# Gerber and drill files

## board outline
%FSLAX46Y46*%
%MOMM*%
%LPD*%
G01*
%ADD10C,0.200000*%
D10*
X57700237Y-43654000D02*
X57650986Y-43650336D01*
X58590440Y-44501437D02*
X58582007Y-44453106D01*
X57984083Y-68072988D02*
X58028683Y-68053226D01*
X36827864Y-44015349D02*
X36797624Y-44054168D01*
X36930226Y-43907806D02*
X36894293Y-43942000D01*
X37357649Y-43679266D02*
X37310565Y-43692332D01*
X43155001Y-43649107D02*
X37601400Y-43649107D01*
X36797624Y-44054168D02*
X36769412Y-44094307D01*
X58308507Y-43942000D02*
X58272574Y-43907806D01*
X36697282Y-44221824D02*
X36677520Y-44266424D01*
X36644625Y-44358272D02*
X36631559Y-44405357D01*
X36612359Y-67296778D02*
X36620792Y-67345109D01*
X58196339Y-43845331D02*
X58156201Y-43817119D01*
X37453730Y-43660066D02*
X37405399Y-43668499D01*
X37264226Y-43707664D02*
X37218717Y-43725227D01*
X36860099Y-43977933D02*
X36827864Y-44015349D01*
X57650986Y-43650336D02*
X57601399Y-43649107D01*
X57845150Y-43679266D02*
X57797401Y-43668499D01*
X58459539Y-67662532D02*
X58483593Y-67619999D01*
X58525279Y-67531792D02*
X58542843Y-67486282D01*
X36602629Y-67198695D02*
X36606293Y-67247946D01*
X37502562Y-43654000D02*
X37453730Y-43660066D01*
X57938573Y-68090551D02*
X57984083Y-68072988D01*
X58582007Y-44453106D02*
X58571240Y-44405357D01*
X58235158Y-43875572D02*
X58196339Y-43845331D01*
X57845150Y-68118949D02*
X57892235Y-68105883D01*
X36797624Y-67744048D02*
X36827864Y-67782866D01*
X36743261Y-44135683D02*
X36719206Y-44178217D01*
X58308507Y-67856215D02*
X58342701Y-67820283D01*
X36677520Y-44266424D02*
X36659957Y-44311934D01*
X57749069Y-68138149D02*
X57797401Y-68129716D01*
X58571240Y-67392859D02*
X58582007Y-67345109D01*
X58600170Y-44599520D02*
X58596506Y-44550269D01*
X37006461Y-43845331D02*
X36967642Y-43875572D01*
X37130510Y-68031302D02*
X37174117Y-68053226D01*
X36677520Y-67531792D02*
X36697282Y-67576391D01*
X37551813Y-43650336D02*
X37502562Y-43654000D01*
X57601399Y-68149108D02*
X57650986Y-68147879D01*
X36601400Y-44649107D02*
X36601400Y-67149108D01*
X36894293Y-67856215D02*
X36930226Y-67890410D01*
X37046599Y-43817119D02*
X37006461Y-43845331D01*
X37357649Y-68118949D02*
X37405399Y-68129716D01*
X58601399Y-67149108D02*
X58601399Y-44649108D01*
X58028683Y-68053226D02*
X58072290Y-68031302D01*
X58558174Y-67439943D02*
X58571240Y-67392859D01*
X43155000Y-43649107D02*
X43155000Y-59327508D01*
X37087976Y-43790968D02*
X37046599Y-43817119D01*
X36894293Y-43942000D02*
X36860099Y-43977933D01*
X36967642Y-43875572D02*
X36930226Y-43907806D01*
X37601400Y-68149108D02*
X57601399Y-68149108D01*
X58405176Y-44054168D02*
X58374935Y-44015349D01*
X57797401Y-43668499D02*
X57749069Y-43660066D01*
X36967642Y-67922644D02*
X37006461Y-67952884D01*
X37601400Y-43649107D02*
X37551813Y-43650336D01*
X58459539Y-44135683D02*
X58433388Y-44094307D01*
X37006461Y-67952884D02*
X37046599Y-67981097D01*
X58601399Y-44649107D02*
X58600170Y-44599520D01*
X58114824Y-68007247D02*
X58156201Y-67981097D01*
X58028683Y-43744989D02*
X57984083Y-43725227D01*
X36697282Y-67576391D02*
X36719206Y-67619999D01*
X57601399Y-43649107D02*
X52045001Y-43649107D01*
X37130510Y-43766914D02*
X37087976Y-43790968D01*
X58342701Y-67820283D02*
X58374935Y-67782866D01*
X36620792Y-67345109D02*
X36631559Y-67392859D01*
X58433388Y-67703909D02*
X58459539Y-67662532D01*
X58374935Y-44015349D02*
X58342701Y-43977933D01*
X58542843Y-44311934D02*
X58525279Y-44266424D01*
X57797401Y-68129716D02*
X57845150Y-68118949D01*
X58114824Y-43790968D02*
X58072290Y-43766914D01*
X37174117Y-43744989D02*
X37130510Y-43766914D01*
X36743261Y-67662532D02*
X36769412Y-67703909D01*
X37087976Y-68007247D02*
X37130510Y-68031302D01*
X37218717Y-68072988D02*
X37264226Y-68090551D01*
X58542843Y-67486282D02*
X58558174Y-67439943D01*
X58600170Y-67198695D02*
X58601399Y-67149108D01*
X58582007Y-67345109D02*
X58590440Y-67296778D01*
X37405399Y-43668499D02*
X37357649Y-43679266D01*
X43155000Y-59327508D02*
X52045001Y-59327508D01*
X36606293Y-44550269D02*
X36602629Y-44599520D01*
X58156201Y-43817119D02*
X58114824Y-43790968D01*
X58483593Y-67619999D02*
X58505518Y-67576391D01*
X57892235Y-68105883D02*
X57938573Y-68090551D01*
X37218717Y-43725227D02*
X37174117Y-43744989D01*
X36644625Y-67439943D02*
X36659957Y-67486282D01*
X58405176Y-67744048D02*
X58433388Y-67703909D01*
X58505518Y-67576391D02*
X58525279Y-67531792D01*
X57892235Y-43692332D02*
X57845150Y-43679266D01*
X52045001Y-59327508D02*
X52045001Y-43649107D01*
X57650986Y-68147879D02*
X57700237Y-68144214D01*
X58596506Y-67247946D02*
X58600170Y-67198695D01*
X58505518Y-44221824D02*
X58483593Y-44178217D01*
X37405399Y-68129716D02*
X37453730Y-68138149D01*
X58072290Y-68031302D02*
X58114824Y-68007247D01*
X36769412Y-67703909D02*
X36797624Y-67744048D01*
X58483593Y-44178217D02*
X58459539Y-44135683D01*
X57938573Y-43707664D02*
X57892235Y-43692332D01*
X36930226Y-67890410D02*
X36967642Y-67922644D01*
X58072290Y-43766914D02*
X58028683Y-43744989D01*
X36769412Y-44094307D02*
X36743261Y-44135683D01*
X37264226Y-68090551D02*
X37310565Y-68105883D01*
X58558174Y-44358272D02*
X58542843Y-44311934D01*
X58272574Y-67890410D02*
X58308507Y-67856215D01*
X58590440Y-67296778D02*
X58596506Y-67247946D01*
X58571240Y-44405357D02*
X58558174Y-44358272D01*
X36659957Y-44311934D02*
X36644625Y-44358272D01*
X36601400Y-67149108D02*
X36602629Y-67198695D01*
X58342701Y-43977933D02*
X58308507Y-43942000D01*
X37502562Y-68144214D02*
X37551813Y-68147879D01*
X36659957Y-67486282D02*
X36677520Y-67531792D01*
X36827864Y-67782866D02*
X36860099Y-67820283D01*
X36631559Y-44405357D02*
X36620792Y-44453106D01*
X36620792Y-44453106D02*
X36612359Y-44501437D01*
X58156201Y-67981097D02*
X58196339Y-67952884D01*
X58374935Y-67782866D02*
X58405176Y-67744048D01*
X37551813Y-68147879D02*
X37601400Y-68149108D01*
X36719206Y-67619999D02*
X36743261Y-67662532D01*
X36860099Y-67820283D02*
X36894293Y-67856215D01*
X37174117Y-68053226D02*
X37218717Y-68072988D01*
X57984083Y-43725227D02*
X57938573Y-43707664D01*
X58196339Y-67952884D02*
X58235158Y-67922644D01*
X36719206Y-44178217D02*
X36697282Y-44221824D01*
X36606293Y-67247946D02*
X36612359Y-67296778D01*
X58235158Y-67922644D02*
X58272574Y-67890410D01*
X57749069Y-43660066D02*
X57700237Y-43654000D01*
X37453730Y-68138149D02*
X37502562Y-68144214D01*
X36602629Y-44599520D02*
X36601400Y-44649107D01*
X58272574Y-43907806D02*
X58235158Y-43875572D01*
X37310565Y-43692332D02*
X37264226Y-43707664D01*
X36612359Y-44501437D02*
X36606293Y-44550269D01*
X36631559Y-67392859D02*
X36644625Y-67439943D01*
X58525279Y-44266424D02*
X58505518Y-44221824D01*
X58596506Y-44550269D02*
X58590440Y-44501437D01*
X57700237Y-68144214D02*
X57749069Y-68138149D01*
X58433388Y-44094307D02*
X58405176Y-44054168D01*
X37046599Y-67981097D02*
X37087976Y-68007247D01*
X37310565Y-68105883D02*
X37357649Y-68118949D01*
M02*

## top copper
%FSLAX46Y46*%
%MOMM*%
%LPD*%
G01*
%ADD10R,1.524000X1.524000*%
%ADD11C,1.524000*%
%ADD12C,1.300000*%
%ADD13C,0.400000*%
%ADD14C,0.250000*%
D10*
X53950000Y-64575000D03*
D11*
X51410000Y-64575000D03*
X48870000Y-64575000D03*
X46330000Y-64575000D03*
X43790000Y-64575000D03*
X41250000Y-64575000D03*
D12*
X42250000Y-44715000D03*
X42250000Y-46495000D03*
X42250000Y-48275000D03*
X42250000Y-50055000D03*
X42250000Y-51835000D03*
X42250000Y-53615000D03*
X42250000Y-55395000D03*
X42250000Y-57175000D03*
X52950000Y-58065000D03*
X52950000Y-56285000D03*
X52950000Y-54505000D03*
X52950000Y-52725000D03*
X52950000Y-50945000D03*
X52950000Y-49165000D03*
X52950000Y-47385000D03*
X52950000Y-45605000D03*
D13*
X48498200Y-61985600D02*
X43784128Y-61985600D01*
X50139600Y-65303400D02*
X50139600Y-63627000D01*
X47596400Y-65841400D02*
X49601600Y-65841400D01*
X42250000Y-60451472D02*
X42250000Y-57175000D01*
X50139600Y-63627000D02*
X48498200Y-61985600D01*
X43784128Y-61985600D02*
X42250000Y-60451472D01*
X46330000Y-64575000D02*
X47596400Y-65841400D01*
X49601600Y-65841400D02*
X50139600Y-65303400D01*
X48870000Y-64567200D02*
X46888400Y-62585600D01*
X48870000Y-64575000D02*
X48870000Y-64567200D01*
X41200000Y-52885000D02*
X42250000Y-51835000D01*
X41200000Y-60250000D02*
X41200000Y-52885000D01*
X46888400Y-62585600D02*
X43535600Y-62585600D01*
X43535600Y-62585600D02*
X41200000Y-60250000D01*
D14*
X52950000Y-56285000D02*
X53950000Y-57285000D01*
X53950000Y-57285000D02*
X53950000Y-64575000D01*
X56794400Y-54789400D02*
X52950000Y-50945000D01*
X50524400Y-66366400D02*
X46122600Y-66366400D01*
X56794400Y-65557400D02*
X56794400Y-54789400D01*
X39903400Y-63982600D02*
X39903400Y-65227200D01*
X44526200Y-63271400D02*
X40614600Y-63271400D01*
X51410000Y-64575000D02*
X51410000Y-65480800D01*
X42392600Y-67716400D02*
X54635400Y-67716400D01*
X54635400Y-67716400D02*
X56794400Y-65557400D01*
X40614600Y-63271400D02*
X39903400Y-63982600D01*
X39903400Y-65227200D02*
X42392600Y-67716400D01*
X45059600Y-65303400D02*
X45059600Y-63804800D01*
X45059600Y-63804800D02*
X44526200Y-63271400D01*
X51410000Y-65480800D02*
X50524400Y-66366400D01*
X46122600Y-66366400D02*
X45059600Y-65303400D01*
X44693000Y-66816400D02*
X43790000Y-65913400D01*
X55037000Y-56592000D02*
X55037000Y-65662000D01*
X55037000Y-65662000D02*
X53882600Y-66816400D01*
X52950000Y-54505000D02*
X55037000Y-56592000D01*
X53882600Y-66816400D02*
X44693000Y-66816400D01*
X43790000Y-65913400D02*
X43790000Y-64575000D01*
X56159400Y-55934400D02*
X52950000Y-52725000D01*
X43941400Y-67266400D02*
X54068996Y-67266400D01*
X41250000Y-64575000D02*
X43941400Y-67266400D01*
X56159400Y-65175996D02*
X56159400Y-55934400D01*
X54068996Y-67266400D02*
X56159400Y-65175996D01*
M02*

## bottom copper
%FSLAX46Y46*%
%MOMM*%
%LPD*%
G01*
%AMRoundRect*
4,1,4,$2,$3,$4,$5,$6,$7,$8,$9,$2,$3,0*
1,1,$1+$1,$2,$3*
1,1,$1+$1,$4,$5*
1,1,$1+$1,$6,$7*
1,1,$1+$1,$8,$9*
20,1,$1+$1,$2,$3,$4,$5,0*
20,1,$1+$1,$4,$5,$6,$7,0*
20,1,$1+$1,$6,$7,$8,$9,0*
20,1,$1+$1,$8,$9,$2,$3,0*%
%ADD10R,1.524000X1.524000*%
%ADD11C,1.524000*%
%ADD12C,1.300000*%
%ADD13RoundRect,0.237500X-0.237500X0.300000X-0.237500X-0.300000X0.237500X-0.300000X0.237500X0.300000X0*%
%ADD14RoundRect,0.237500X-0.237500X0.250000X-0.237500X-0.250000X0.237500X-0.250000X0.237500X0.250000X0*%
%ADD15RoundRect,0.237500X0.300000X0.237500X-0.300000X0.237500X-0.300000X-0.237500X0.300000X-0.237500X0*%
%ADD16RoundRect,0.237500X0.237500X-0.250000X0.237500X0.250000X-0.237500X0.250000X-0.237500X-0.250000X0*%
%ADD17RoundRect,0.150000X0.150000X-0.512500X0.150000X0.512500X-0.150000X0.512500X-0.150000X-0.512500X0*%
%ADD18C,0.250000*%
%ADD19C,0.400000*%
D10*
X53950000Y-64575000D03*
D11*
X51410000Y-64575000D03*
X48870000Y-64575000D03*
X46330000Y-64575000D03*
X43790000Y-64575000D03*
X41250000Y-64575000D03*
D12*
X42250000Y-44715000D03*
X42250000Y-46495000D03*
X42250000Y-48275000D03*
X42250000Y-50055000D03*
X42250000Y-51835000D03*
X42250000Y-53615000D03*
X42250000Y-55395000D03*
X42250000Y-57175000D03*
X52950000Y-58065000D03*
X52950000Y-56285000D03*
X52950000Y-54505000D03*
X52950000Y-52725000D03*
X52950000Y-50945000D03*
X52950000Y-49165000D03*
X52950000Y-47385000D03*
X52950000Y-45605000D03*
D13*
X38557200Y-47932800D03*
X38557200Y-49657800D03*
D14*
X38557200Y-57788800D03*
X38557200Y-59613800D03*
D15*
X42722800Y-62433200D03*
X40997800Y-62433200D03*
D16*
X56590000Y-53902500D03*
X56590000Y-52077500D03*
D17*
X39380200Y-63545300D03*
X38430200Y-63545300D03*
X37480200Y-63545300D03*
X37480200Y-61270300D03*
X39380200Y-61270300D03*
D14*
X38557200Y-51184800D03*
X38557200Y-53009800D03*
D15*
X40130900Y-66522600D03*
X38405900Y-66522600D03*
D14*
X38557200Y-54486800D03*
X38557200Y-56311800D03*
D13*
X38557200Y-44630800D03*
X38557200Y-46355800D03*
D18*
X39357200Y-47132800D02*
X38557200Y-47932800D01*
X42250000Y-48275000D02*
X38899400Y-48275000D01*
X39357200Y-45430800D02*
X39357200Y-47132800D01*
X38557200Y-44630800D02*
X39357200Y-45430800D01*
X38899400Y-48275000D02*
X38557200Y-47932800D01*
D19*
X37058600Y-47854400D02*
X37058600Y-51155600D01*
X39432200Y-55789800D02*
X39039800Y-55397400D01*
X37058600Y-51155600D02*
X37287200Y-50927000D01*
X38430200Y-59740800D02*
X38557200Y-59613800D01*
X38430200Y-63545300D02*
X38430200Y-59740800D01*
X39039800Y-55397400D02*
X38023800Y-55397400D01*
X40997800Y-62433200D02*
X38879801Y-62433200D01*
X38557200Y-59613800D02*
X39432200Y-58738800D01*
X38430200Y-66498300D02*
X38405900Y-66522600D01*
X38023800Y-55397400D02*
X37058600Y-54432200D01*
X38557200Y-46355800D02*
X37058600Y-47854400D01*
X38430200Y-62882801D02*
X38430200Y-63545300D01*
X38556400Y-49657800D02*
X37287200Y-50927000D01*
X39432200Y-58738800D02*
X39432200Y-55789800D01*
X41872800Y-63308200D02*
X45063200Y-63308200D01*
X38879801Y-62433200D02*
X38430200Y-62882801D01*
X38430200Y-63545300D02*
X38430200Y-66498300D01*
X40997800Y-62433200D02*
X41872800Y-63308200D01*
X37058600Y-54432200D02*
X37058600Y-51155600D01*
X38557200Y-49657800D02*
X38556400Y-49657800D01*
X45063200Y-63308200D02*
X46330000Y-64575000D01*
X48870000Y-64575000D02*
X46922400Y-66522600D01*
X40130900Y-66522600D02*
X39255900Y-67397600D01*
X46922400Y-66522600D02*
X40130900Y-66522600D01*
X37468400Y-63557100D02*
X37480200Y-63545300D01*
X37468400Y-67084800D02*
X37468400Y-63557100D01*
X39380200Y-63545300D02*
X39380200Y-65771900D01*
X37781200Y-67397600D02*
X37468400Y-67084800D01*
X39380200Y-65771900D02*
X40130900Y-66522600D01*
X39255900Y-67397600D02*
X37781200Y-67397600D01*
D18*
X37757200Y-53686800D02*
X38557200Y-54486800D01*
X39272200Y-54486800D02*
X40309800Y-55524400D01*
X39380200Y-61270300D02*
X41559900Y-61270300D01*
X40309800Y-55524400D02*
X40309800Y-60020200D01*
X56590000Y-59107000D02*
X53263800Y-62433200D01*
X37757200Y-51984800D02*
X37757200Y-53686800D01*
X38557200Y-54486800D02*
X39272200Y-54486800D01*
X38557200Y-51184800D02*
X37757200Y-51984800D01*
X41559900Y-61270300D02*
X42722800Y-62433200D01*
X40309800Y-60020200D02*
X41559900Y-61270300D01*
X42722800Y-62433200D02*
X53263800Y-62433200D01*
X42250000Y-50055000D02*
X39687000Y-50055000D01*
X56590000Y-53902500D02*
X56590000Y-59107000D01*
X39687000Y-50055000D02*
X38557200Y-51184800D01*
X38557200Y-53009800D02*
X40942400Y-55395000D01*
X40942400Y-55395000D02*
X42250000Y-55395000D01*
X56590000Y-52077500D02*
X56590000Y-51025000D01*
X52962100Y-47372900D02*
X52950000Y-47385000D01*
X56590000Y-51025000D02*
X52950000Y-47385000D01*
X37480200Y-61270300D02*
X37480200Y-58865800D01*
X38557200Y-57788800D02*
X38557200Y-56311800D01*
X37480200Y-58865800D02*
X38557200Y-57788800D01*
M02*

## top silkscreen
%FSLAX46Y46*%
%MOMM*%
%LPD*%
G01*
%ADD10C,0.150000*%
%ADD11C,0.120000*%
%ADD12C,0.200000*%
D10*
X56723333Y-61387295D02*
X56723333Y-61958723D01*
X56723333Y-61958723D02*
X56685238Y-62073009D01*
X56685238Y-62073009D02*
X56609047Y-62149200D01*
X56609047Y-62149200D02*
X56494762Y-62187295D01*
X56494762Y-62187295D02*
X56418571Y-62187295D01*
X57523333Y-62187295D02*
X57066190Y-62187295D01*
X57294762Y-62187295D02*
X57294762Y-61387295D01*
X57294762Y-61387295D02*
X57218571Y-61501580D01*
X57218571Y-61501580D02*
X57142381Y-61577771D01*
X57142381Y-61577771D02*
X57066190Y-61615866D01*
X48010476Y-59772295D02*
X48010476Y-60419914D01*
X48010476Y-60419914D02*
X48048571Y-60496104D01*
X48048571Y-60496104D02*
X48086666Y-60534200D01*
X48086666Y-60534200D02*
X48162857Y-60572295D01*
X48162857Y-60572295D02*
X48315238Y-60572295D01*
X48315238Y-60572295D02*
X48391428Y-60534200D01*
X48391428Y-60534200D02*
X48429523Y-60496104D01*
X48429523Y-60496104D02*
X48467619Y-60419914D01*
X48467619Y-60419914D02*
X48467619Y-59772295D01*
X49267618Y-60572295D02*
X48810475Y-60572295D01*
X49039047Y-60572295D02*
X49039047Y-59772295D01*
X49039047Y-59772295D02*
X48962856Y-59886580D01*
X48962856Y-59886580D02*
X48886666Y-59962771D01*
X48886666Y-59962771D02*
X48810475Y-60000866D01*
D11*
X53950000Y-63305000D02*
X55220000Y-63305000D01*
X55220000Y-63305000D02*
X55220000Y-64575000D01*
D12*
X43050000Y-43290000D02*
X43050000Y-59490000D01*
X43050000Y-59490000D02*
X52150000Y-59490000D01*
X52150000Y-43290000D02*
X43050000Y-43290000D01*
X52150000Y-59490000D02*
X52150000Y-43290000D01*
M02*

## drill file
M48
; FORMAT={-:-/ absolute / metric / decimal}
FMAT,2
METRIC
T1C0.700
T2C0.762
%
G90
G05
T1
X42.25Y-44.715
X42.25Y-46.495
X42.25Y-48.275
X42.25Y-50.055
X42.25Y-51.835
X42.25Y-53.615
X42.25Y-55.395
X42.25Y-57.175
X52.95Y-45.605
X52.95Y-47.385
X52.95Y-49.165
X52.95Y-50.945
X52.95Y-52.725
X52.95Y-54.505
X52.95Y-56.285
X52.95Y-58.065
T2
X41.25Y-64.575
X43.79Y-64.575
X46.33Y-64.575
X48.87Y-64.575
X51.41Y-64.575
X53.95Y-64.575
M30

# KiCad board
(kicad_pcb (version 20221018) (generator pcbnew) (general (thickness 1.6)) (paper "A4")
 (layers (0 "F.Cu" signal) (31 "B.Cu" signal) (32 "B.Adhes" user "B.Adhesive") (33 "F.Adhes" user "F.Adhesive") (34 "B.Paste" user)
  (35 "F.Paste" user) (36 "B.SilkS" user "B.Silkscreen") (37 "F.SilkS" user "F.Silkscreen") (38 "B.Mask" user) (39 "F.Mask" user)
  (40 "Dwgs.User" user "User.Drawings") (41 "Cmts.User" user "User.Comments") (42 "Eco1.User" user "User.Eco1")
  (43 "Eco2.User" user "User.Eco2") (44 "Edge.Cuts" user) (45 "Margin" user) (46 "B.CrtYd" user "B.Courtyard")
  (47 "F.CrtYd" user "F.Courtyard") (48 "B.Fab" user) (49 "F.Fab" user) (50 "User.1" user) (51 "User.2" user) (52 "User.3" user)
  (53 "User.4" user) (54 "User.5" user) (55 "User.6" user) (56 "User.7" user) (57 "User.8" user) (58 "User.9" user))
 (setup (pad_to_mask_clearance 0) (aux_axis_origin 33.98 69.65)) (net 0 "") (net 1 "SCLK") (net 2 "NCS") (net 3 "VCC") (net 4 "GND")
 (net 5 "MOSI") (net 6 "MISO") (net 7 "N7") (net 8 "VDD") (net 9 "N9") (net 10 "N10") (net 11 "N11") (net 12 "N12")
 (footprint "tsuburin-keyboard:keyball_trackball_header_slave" (layer "F.Cu") (at 43.59 62.995)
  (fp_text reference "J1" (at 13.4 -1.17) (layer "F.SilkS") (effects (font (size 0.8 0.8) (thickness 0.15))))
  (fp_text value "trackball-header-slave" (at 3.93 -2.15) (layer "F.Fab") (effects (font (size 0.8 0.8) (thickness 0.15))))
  (fp_line (start 10.36 0.31) (end 11.63 0.31) (stroke (width 0.12) (type solid)) (layer "F.SilkS"))
  (fp_line (start 11.63 0.31) (end 11.63 1.58) (stroke (width 0.12) (type solid)) (layer "F.SilkS"))
  (pad "1" thru_hole rect (at 10.36 1.58 270) (size 1.524 1.524) (drill 0.762) (layers "*.Cu" "*.Mask") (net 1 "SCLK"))
  (pad "2" thru_hole circle (at 7.82 1.58 270) (size 1.524 1.524) (drill 0.762) (layers "*.Cu" "*.Mask") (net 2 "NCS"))
  (pad "3" thru_hole circle (at 5.28 1.58 270) (size 1.524 1.524) (drill 0.762) (layers "*.Cu" "*.Mask") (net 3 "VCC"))
  (pad "4" thru_hole circle (at 2.74 1.58 270) (size 1.524 1.524) (drill 0.762) (layers "*.Cu" "*.Mask") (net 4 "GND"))
  (pad "5" thru_hole circle (at 0.2 1.58 270) (size 1.524 1.524) (drill 0.762) (layers "*.Cu" "*.Mask") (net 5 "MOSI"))
  (pad "6" thru_hole circle (at -2.34 1.58 270) (size 1.524 1.524) (drill 0.762) (layers "*.Cu" "*.Mask") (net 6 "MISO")))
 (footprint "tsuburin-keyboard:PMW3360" (layer "F.Cu") (at 47.6 51.39)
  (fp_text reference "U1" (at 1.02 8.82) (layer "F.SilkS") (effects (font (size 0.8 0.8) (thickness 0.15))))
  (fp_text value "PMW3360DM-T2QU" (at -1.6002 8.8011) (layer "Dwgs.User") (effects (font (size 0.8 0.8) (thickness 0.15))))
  (fp_line (start -4.55 -8.1) (end -4.55 8.1) (stroke (width 0.2) (type solid)) (layer "F.SilkS"))
  (fp_line (start -4.55 8.1) (end 4.55 8.1) (stroke (width 0.2) (type solid)) (layer "F.SilkS"))
  (fp_line (start 4.55 -8.1) (end -4.55 -8.1) (stroke (width 0.2) (type solid)) (layer "F.SilkS"))
  (fp_line (start 4.55 8.1) (end 4.55 -8.1) (stroke (width 0.2) (type solid)) (layer "F.SilkS"))
  (pad "1" thru_hole circle (at -5.35 -6.675) (size 1.3 1.3) (drill 0.7) (layers "*.Cu" "*.Mask") (solder_mask_margin 0.102))
  (pad "2" thru_hole circle (at -5.35 -4.895) (size 1.3 1.3) (drill 0.7) (layers "*.Cu" "*.Mask") (solder_mask_margin 0.102))
  (pad "3" thru_hole circle (at -5.35 -3.115) (size 1.3 1.3) (drill 0.7) (layers "*.Cu" "*.Mask") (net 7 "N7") (solder_mask_margin 0.102))
  (pad "4" thru_hole circle (at -5.35 -1.335) (size 1.3 1.3) (drill 0.7) (layers "*.Cu" "*.Mask") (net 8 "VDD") (solder_mask_margin 0.102))
  (pad "5" thru_hole circle (at -5.35 0.445) (size 1.3 1.3) (drill 0.7) (layers "*.Cu" "*.Mask") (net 3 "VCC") (solder_mask_margin 0.102))
  (pad "6" thru_hole circle (at -5.35 2.225) (size 1.3 1.3) (drill 0.7) (layers "*.Cu" "*.Mask") (solder_mask_margin 0.102))
  (pad "7" thru_hole circle (at -5.35 4.005) (size 1.3 1.3) (drill 0.7) (layers "*.Cu" "*.Mask") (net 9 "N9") (solder_mask_margin 0.102))
  (pad "8" thru_hole circle (at -5.35 5.785) (size 1.3 1.3) (drill 0.7) (layers "*.Cu" "*.Mask") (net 4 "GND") (solder_mask_margin 0.102))
  (pad "9" thru_hole circle (at 5.35 6.675) (size 1.3 1.3) (drill 0.7) (layers "*.Cu" "*.Mask") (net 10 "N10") (solder_mask_margin 0.102))
  (pad "10" thru_hole circle (at 5.35 4.895) (size 1.3 1.3) (drill 0.7) (layers "*.Cu" "*.Mask") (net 1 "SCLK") (solder_mask_margin 0.102))
  (pad "11" thru_hole circle (at 5.35 3.115) (size 1.3 1.3) (drill 0.7) (layers "*.Cu" "*.Mask") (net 5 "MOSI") (solder_mask_margin 0.102))
  (pad "12" thru_hole circle (at 5.35 1.335) (size 1.3 1.3) (drill 0.7) (layers "*.Cu" "*.Mask") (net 6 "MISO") (solder_mask_margin 0.102))
  (pad "13" thru_hole circle (at 5.35 -0.445) (size 1.3 1.3) (drill 0.7) (layers "*.Cu" "*.Mask") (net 2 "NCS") (solder_mask_margin 0.102))
  (pad "14" thru_hole circle (at 5.35 -2.225) (size 1.3 1.3) (drill 0.7) (layers "*.Cu" "*.Mask") (solder_mask_margin 0.102))
  (pad "15" thru_hole circle (at 5.35 -4.005) (size 1.3 1.3) (drill 0.7) (layers "*.Cu" "*.Mask") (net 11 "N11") (solder_mask_margin 0.102))
  (pad "16" thru_hole circle (at 5.35 -5.785) (size 1.3 1.3) (drill 0.7) (layers "*.Cu" "*.Mask") (solder_mask_margin 0.102))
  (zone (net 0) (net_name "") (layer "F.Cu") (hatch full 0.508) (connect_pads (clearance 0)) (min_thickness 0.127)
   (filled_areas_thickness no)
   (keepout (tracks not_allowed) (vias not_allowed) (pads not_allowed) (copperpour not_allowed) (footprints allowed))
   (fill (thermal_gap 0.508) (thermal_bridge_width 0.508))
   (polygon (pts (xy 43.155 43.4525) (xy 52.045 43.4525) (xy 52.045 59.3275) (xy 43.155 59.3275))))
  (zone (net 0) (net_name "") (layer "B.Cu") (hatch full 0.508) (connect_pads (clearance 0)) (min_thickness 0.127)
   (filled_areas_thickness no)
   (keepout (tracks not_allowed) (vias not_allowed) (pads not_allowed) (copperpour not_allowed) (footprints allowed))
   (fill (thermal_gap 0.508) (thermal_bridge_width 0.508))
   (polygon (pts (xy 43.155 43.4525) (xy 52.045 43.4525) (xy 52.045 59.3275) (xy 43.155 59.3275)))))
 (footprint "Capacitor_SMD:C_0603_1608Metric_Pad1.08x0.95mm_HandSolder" (layer "B.Cu") (at 38.5572 48.7953 -90)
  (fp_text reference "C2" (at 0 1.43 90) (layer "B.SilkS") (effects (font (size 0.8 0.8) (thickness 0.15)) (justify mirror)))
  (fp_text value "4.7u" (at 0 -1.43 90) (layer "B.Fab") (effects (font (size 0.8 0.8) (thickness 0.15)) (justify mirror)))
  (pad "1" smd roundrect (at -0.8625 0 270) (size 1.075 0.95) (layers "B.Cu" "B.Paste" "B.Mask") (roundrect_rratio 0.25) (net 7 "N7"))
  (pad "2" smd roundrect (at 0.8625 0 270) (size 1.075 0.95) (layers "B.Cu" "B.Paste" "B.Mask") (roundrect_rratio 0.25) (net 4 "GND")))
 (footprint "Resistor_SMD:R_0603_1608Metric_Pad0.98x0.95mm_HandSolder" (layer "B.Cu") (at 38.5572 58.7013 -90)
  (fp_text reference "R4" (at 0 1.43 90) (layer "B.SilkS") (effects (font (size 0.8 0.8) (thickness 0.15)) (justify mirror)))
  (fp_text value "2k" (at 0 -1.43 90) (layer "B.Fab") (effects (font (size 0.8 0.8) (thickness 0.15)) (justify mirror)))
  (pad "1" smd roundrect (at -0.9125 0 270) (size 0.975 0.95) (layers "B.Cu" "B.Paste" "B.Mask") (roundrect_rratio 0.25) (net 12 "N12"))
  (pad "2" smd roundrect (at 0.9125 0 270) (size 0.975 0.95) (layers "B.Cu" "B.Paste" "B.Mask") (roundrect_rratio 0.25) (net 4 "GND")))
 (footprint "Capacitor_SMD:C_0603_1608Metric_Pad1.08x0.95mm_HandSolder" (layer "B.Cu") (at 41.8603 62.4332 180)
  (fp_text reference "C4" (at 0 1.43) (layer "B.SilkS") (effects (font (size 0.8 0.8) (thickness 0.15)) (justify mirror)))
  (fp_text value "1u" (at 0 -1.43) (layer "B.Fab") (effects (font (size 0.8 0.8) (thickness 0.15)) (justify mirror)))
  (pad "1" smd roundrect (at -0.8625 0 180) (size 1.075 0.95) (layers "B.Cu" "B.Paste" "B.Mask") (roundrect_rratio 0.25) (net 8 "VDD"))
  (pad "2" smd roundrect (at 0.8625 0 180) (size 1.075 0.95) (layers "B.Cu" "B.Paste" "B.Mask") (roundrect_rratio 0.25) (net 4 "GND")))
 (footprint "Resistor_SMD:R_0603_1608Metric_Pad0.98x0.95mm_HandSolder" (layer "B.Cu") (at 56.59 52.99 90)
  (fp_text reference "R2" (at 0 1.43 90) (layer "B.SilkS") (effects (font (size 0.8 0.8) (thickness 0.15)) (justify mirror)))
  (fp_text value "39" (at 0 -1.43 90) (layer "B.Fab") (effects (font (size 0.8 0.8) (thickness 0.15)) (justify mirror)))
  (pad "1" smd roundrect (at -0.9125 0 90) (size 0.975 0.95) (layers "B.Cu" "B.Paste" "B.Mask") (roundrect_rratio 0.25) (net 8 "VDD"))
  (pad "2" smd roundrect (at 0.9125 0 90) (size 0.975 0.95) (layers "B.Cu" "B.Paste" "B.Mask") (roundrect_rratio 0.25) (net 11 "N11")))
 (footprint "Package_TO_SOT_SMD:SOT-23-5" (layer "B.Cu") (at 38.4302 62.4078 90)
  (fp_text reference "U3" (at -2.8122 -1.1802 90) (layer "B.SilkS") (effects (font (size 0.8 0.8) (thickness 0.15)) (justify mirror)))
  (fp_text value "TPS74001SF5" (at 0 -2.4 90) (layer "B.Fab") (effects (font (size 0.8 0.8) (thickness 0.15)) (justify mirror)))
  (pad "1" smd roundrect (at -1.1375 0.95 90) (size 1.325 0.6) (layers "B.Cu" "B.Paste" "B.Mask") (roundrect_rratio 0.25) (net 3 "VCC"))
  (pad "2" smd roundrect (at -1.1375 0 90) (size 1.325 0.6) (layers "B.Cu" "B.Paste" "B.Mask") (roundrect_rratio 0.25) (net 4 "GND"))
  (pad "3" smd roundrect (at -1.1375 -0.95 90) (size 1.325 0.6) (layers "B.Cu" "B.Paste" "B.Mask") (roundrect_rratio 0.25) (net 3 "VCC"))
  (pad "4" smd roundrect (at 1.1375 -0.95 90) (size 1.325 0.6) (layers "B.Cu" "B.Paste" "B.Mask") (roundrect_rratio 0.25) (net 12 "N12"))
  (pad "5" smd roundrect (at 1.1375 0.95 90) (size 1.325 0.6) (layers "B.Cu" "B.Paste" "B.Mask") (roundrect_rratio 0.25) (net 8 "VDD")))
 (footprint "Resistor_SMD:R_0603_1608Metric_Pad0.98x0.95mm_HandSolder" (layer "B.Cu") (at 38.5572 52.0973 -90)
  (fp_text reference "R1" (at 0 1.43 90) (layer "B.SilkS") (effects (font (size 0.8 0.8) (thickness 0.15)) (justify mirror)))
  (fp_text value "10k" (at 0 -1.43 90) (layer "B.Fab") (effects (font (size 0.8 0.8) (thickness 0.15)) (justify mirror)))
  (pad "1" smd roundrect (at -0.9125 0 270) (size 0.975 0.95) (layers "B.Cu" "B.Paste" "B.Mask") (roundrect_rratio 0.25) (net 8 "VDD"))
  (pad "2" smd roundrect (at 0.9125 0 270) (size 0.975 0.95) (layers "B.Cu" "B.Paste" "B.Mask") (roundrect_rratio 0.25) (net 9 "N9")))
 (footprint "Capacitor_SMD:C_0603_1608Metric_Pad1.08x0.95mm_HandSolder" (layer "B.Cu") (at 39.2684 66.5226 180)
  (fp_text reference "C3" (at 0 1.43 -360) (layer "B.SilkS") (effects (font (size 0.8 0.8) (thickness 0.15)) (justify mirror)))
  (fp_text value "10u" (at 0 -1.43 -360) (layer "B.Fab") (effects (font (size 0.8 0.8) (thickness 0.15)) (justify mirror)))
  (pad "1" smd roundrect (at -0.8625 0 180) (size 1.075 0.95) (layers "B.Cu" "B.Paste" "B.Mask") (roundrect_rratio 0.25) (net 3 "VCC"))
  (pad "2" smd roundrect (at 0.8625 0 180) (size 1.075 0.95) (layers "B.Cu" "B.Paste" "B.Mask") (roundrect_rratio 0.25) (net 4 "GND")))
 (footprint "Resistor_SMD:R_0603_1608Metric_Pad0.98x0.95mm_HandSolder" (layer "B.Cu") (at 38.5572 55.3993 -90)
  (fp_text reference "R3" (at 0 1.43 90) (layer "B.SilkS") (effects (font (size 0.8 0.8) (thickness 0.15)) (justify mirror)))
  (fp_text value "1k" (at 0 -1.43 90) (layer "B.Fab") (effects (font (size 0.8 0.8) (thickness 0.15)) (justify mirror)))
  (pad "1" smd roundrect (at -0.9125 0 270) (size 0.975 0.95) (layers "B.Cu" "B.Paste" "B.Mask") (roundrect_rratio 0.25) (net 8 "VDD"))
  (pad "2" smd roundrect (at 0.9125 0 270) (size 0.975 0.95) (layers "B.Cu" "B.Paste" "B.Mask") (roundrect_rratio 0.25) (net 12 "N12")))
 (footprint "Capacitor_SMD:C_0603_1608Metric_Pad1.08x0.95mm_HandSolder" (layer "B.Cu") (at 38.5572 45.4933 -90)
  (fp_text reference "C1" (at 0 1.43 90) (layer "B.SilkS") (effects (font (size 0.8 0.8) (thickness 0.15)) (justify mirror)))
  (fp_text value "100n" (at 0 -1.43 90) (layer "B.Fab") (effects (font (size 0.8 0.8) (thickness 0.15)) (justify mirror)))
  (pad "1" smd roundrect (at -0.8625 0 270) (size 1.075 0.95) (layers "B.Cu" "B.Paste" "B.Mask") (roundrect_rratio 0.25) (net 7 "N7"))
  (pad "2" smd roundrect (at 0.8625 0 270) (size 1.075 0.95) (layers "B.Cu" "B.Paste" "B.Mask") (roundrect_rratio 0.25) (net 4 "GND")))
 (gr_line (start 57.700237 43.654) (end 57.650986 43.650336) (stroke (width 0.2) (type solid)) (layer "Edge.Cuts"))
 (gr_line (start 58.59044 44.501437) (end 58.582007 44.453106) (stroke (width 0.2) (type solid)) (layer "Edge.Cuts"))
 (gr_line (start 57.984083 68.072988) (end 58.028683 68.053226) (stroke (width 0.2) (type solid)) (layer "Edge.Cuts"))
 (gr_line (start 36.827864 44.015349) (end 36.797624 44.054168) (stroke (width 0.2) (type solid)) (layer "Edge.Cuts"))
 (gr_line (start 36.930226 43.907806) (end 36.894293 43.942) (stroke (width 0.2) (type solid)) (layer "Edge.Cuts"))
 (gr_line (start 37.357649 43.679266) (end 37.310565 43.692332) (stroke (width 0.2) (type solid)) (layer "Edge.Cuts"))
 (gr_line (start 43.155001 43.649107) (end 37.6014 43.649107) (stroke (width 0.2) (type solid)) (layer "Edge.Cuts"))
 (gr_line (start 36.797624 44.054168) (end 36.769412 44.094307) (stroke (width 0.2) (type solid)) (layer "Edge.Cuts"))
 (gr_line (start 58.308507 43.942) (end 58.272574 43.907806) (stroke (width 0.2) (type solid)) (layer "Edge.Cuts"))
 (gr_line (start 36.697282 44.221824) (end 36.67752 44.266424) (stroke (width 0.2) (type solid)) (layer "Edge.Cuts"))
 (gr_line (start 36.644625 44.358272) (end 36.631559 44.405357) (stroke (width 0.2) (type solid)) (layer "Edge.Cuts"))
 (gr_line (start 36.612359 67.296778) (end 36.620792 67.345109) (stroke (width 0.2) (type solid)) (layer "Edge.Cuts"))
 (gr_line (start 58.196339 43.845331) (end 58.156201 43.817119) (stroke (width 0.2) (type solid)) (layer "Edge.Cuts"))
 (gr_line (start 37.45373 43.660066) (end 37.405399 43.668499) (stroke (width 0.2) (type solid)) (layer "Edge.Cuts"))
 (gr_line (start 37.264226 43.707664) (end 37.218717 43.725227) (stroke (width 0.2) (type solid)) (layer "Edge.Cuts"))
 (gr_line (start 36.860099 43.977933) (end 36.827864 44.015349) (stroke (width 0.2) (type solid)) (layer "Edge.Cuts"))
 (gr_line (start 57.650986 43.650336) (end 57.601399 43.649107) (stroke (width 0.2) (type solid)) (layer "Edge.Cuts"))
 (gr_line (start 57.84515 43.679266) (end 57.797401 43.668499) (stroke (width 0.2) (type solid)) (layer "Edge.Cuts"))
 (gr_line (start 58.459539 67.662532) (end 58.483593 67.619999) (stroke (width 0.2) (type solid)) (layer "Edge.Cuts"))
 (gr_line (start 58.525279 67.531792) (end 58.542843 67.486282) (stroke (width 0.2) (type solid)) (layer "Edge.Cuts"))
 (gr_line (start 36.602629 67.198695) (end 36.606293 67.247946) (stroke (width 0.2) (type solid)) (layer "Edge.Cuts"))
 (gr_line (start 37.502562 43.654) (end 37.45373 43.660066) (stroke (width 0.2) (type solid)) (layer "Edge.Cuts"))
 (gr_line (start 57.938573 68.090551) (end 57.984083 68.072988) (stroke (width 0.2) (type solid)) (layer "Edge.Cuts"))
 (gr_line (start 58.582007 44.453106) (end 58.57124 44.405357) (stroke (width 0.2) (type solid)) (layer "Edge.Cuts"))
 (gr_line (start 58.235158 43.875572) (end 58.196339 43.845331) (stroke (width 0.2) (type solid)) (layer "Edge.Cuts"))
 (gr_line (start 57.84515 68.118949) (end 57.892235 68.105883) (stroke (width 0.2) (type solid)) (layer "Edge.Cuts"))
 (gr_line (start 36.797624 67.744048) (end 36.827864 67.782866) (stroke (width 0.2) (type solid)) (layer "Edge.Cuts"))
 (gr_line (start 36.743261 44.135683) (end 36.719206 44.178217) (stroke (width 0.2) (type solid)) (layer "Edge.Cuts"))
 (gr_line (start 58.308507 67.856215) (end 58.342701 67.820283) (stroke (width 0.2) (type solid)) (layer "Edge.Cuts"))
 (gr_line (start 36.67752 44.266424) (end 36.659957 44.311934) (stroke (width 0.2) (type solid)) (layer "Edge.Cuts"))
 (gr_line (start 57.749069 68.138149) (end 57.797401 68.129716) (stroke (width 0.2) (type solid)) (layer "Edge.Cuts"))
 (gr_line (start 58.57124 67.392859) (end 58.582007 67.345109) (stroke (width 0.2) (type solid)) (layer "Edge.Cuts"))
 (gr_line (start 58.60017 44.59952) (end 58.596506 44.550269) (stroke (width 0.2) (type solid)) (layer "Edge.Cuts"))
 (gr_line (start 37.006461 43.845331) (end 36.967642 43.875572) (stroke (width 0.2) (type solid)) (layer "Edge.Cuts"))
 (gr_line (start 37.13051 68.031302) (end 37.174117 68.053226) (stroke (width 0.2) (type solid)) (layer "Edge.Cuts"))
 (gr_line (start 36.67752 67.531792) (end 36.697282 67.576391) (stroke (width 0.2) (type solid)) (layer "Edge.Cuts"))
 (gr_line (start 37.551813 43.650336) (end 37.502562 43.654) (stroke (width 0.2) (type solid)) (layer "Edge.Cuts"))
 (gr_line (start 57.601399 68.149108) (end 57.650986 68.147879) (stroke (width 0.2) (type solid)) (layer "Edge.Cuts"))
 (gr_line (start 36.6014 44.649107) (end 36.6014 67.149108) (stroke (width 0.2) (type solid)) (layer "Edge.Cuts"))
 (gr_line (start 36.894293 67.856215) (end 36.930226 67.89041) (stroke (width 0.2) (type solid)) (layer "Edge.Cuts"))
 (gr_line (start 37.046599 43.817119) (end 37.006461 43.845331) (stroke (width 0.2) (type solid)) (layer "Edge.Cuts"))
 (gr_line (start 37.357649 68.118949) (end 37.405399 68.129716) (stroke (width 0.2) (type solid)) (layer "Edge.Cuts"))
 (gr_line (start 58.601399 67.149108) (end 58.601399 44.649108) (stroke (width 0.2) (type solid)) (layer "Edge.Cuts"))
 (gr_line (start 58.028683 68.053226) (end 58.07229 68.031302) (stroke (width 0.2) (type solid)) (layer "Edge.Cuts"))
 (gr_line (start 58.558174 67.439943) (end 58.57124 67.392859) (stroke (width 0.2) (type solid)) (layer "Edge.Cuts"))
 (gr_line (start 43.155 43.649107) (end 43.155 59.327508) (stroke (width 0.2) (type solid)) (layer "Edge.Cuts"))
 (gr_line (start 37.087976 43.790968) (end 37.046599 43.817119) (stroke (width 0.2) (type solid)) (layer "Edge.Cuts"))
 (gr_line (start 36.894293 43.942) (end 36.860099 43.977933) (stroke (width 0.2) (type solid)) (layer "Edge.Cuts"))
 (gr_line (start 36.967642 43.875572) (end 36.930226 43.907806) (stroke (width 0.2) (type solid)) (layer "Edge.Cuts"))
 (gr_line (start 37.6014 68.149108) (end 57.601399 68.149108) (stroke (width 0.2) (type solid)) (layer "Edge.Cuts"))
 (gr_line (start 58.405176 44.054168) (end 58.374935 44.015349) (stroke (width 0.2) (type solid)) (layer "Edge.Cuts"))
 (gr_line (start 57.797401 43.668499) (end 57.749069 43.660066) (stroke (width 0.2) (type solid)) (layer "Edge.Cuts"))
 (gr_line (start 36.967642 67.922644) (end 37.006461 67.952884) (stroke (width 0.2) (type solid)) (layer "Edge.Cuts"))
 (gr_line (start 37.6014 43.649107) (end 37.551813 43.650336) (stroke (width 0.2) (type solid)) (layer "Edge.Cuts"))
 (gr_line (start 58.459539 44.135683) (end 58.433388 44.094307) (stroke (width 0.2) (type solid)) (layer "Edge.Cuts"))
 (gr_line (start 37.006461 67.952884) (end 37.046599 67.981097) (stroke (width 0.2) (type solid)) (layer "Edge.Cuts"))
 (gr_line (start 58.601399 44.649107) (end 58.60017 44.59952) (stroke (width 0.2) (type solid)) (layer "Edge.Cuts"))
 (gr_line (start 58.114824 68.007247) (end 58.156201 67.981097) (stroke (width 0.2) (type solid)) (layer "Edge.Cuts"))
 (gr_line (start 58.028683 43.744989) (end 57.984083 43.725227) (stroke (width 0.2) (type solid)) (layer "Edge.Cuts"))
 (gr_line (start 36.697282 67.576391) (end 36.719206 67.619999) (stroke (width 0.2) (type solid)) (layer "Edge.Cuts"))
 (gr_line (start 57.601399 43.649107) (end 52.045001 43.649107) (stroke (width 0.2) (type solid)) (layer "Edge.Cuts"))
 (gr_line (start 37.13051 43.766914) (end 37.087976 43.790968) (stroke (width 0.2) (type solid)) (layer "Edge.Cuts"))
 (gr_line (start 58.342701 67.820283) (end 58.374935 67.782866) (stroke (width 0.2) (type solid)) (layer "Edge.Cuts"))
 (gr_line (start 36.620792 67.345109) (end 36.631559 67.392859) (stroke (width 0.2) (type solid)) (layer "Edge.Cuts"))
 (gr_line (start 58.433388 67.703909) (end 58.459539 67.662532) (stroke (width 0.2) (type solid)) (layer "Edge.Cuts"))
 (gr_line (start 58.374935 44.015349) (end 58.342701 43.977933) (stroke (width 0.2) (type solid)) (layer "Edge.Cuts"))
 (gr_line (start 58.542843 44.311934) (end 58.525279 44.266424) (stroke (width 0.2) (type solid)) (layer "Edge.Cuts"))
 (gr_line (start 57.797401 68.129716) (end 57.84515 68.118949) (stroke (width 0.2) (type solid)) (layer "Edge.Cuts"))
 (gr_line (start 58.114824 43.790968) (end 58.07229 43.766914) (stroke (width 0.2) (type solid)) (layer "Edge.Cuts"))
 (gr_line (start 37.174117 43.744989) (end 37.13051 43.766914) (stroke (width 0.2) (type solid)) (layer "Edge.Cuts"))
 (gr_line (start 36.743261 67.662532) (end 36.769412 67.703909) (stroke (width 0.2) (type solid)) (layer "Edge.Cuts"))
 (gr_line (start 37.087976 68.007247) (end 37.13051 68.031302) (stroke (width 0.2) (type solid)) (layer "Edge.Cuts"))
 (gr_line (start 37.218717 68.072988) (end 37.264226 68.090551) (stroke (width 0.2) (type solid)) (layer "Edge.Cuts"))
 (gr_line (start 58.542843 67.486282) (end 58.558174 67.439943) (stroke (width 0.2) (type solid)) (layer "Edge.Cuts"))
 (gr_line (start 58.60017 67.198695) (end 58.601399 67.149108) (stroke (width 0.2) (type solid)) (layer "Edge.Cuts"))
 (gr_line (start 58.582007 67.345109) (end 58.59044 67.296778) (stroke (width 0.2) (type solid)) (layer "Edge.Cuts"))
 (gr_line (start 37.405399 43.668499) (end 37.357649 43.679266) (stroke (width 0.2) (type solid)) (layer "Edge.Cuts"))
 (gr_line (start 43.155 59.327508) (end 52.045001 59.327508) (stroke (width 0.2) (type solid)) (layer "Edge.Cuts"))
 (gr_line (start 36.606293 44.550269) (end 36.602629 44.59952) (stroke (width 0.2) (type solid)) (layer "Edge.Cuts"))
 (gr_line (start 58.156201 43.817119) (end 58.114824 43.790968) (stroke (width 0.2) (type solid)) (layer "Edge.Cuts"))
 (gr_line (start 58.483593 67.619999) (end 58.505518 67.576391) (stroke (width 0.2) (type solid)) (layer "Edge.Cuts"))
 (gr_line (start 57.892235 68.105883) (end 57.938573 68.090551) (stroke (width 0.2) (type solid)) (layer "Edge.Cuts"))
 (gr_line (start 37.218717 43.725227) (end 37.174117 43.744989) (stroke (width 0.2) (type solid)) (layer "Edge.Cuts"))
 (gr_line (start 36.644625 67.439943) (end 36.659957 67.486282) (stroke (width 0.2) (type solid)) (layer "Edge.Cuts"))
 (gr_line (start 58.405176 67.744048) (end 58.433388 67.703909) (stroke (width 0.2) (type solid)) (layer "Edge.Cuts"))
 (gr_line (start 58.505518 67.576391) (end 58.525279 67.531792) (stroke (width 0.2) (type solid)) (layer "Edge.Cuts"))
 (gr_line (start 57.892235 43.692332) (end 57.84515 43.679266) (stroke (width 0.2) (type solid)) (layer "Edge.Cuts"))
 (gr_line (start 52.045001 59.327508) (end 52.045001 43.649107) (stroke (width 0.2) (type solid)) (layer "Edge.Cuts"))
 (gr_line (start 57.650986 68.147879) (end 57.700237 68.144214) (stroke (width 0.2) (type solid)) (layer "Edge.Cuts"))
 (gr_line (start 58.596506 67.247946) (end 58.60017 67.198695) (stroke (width 0.2) (type solid)) (layer "Edge.Cuts"))
 (gr_line (start 58.505518 44.221824) (end 58.483593 44.178217) (stroke (width 0.2) (type solid)) (layer "Edge.Cuts"))
 (gr_line (start 37.405399 68.129716) (end 37.45373 68.138149) (stroke (width 0.2) (type solid)) (layer "Edge.Cuts"))
 (gr_line (start 58.07229 68.031302) (end 58.114824 68.007247) (stroke (width 0.2) (type solid)) (layer "Edge.Cuts"))
 (gr_line (start 36.769412 67.703909) (end 36.797624 67.744048) (stroke (width 0.2) (type solid)) (layer "Edge.Cuts"))
 (gr_line (start 58.483593 44.178217) (end 58.459539 44.135683) (stroke (width 0.2) (type solid)) (layer "Edge.Cuts"))
 (gr_line (start 57.938573 43.707664) (end 57.892235 43.692332) (stroke (width 0.2) (type solid)) (layer "Edge.Cuts"))
 (gr_line (start 36.930226 67.89041) (end 36.967642 67.922644) (stroke (width 0.2) (type solid)) (layer "Edge.Cuts"))
 (gr_line (start 58.07229 43.766914) (end 58.028683 43.744989) (stroke (width 0.2) (type solid)) (layer "Edge.Cuts"))
 (gr_line (start 36.769412 44.094307) (end 36.743261 44.135683) (stroke (width 0.2) (type solid)) (layer "Edge.Cuts"))
 (gr_line (start 37.264226 68.090551) (end 37.310565 68.105883) (stroke (width 0.2) (type solid)) (layer "Edge.Cuts"))
 (gr_line (start 58.558174 44.358272) (end 58.542843 44.311934) (stroke (width 0.2) (type solid)) (layer "Edge.Cuts"))
 (gr_line (start 58.272574 67.89041) (end 58.308507 67.856215) (stroke (width 0.2) (type solid)) (layer "Edge.Cuts"))
 (gr_line (start 58.59044 67.296778) (end 58.596506 67.247946) (stroke (width 0.2) (type solid)) (layer "Edge.Cuts"))
 (gr_line (start 58.57124 44.405357) (end 58.558174 44.358272) (stroke (width 0.2) (type solid)) (layer "Edge.Cuts"))
 (gr_line (start 36.659957 44.311934) (end 36.644625 44.358272) (stroke (width 0.2) (type solid)) (layer "Edge.Cuts"))
 (gr_line (start 36.6014 67.149108) (end 36.602629 67.198695) (stroke (width 0.2) (type solid)) (layer "Edge.Cuts"))
 (gr_line (start 58.342701 43.977933) (end 58.308507 43.942) (stroke (width 0.2) (type solid)) (layer "Edge.Cuts"))
 (gr_line (start 37.502562 68.144214) (end 37.551813 68.147879) (stroke (width 0.2) (type solid)) (layer "Edge.Cuts"))
 (gr_line (start 36.659957 67.486282) (end 36.67752 67.531792) (stroke (width 0.2) (type solid)) (layer "Edge.Cuts"))
 (gr_line (start 36.827864 67.782866) (end 36.860099 67.820283) (stroke (width 0.2) (type solid)) (layer "Edge.Cuts"))
 (gr_line (start 36.631559 44.405357) (end 36.620792 44.453106) (stroke (width 0.2) (type solid)) (layer "Edge.Cuts"))
 (gr_line (start 36.620792 44.453106) (end 36.612359 44.501437) (stroke (width 0.2) (type solid)) (layer "Edge.Cuts"))
 (gr_line (start 58.156201 67.981097) (end 58.196339 67.952884) (stroke (width 0.2) (type solid)) (layer "Edge.Cuts"))
 (gr_line (start 58.374935 67.782866) (end 58.405176 67.744048) (stroke (width 0.2) (type solid)) (layer "Edge.Cuts"))
 (gr_line (start 37.551813 68.147879) (end 37.6014 68.149108) (stroke (width 0.2) (type solid)) (layer "Edge.Cuts"))
 (gr_line (start 36.719206 67.619999) (end 36.743261 67.662532) (stroke (width 0.2) (type solid)) (layer "Edge.Cuts"))
 (gr_line (start 36.860099 67.820283) (end 36.894293 67.856215) (stroke (width 0.2) (type solid)) (layer "Edge.Cuts"))
 (gr_line (start 37.174117 68.053226) (end 37.218717 68.072988) (stroke (width 0.2) (type solid)) (layer "Edge.Cuts"))
 (gr_line (start 57.984083 43.725227) (end 57.938573 43.707664) (stroke (width 0.2) (type solid)) (layer "Edge.Cuts"))
 (gr_line (start 58.196339 67.952884) (end 58.235158 67.922644) (stroke (width 0.2) (type solid)) (layer "Edge.Cuts"))
 (gr_line (start 36.719206 44.178217) (end 36.697282 44.221824) (stroke (width 0.2) (type solid)) (layer "Edge.Cuts"))
 (gr_line (start 36.606293 67.247946) (end 36.612359 67.296778) (stroke (width 0.2) (type solid)) (layer "Edge.Cuts"))
 (gr_line (start 58.235158 67.922644) (end 58.272574 67.89041) (stroke (width 0.2) (type solid)) (layer "Edge.Cuts"))
 (gr_line (start 57.749069 43.660066) (end 57.700237 43.654) (stroke (width 0.2) (type solid)) (layer "Edge.Cuts"))
 (gr_line (start 37.45373 68.138149) (end 37.502562 68.144214) (stroke (width 0.2) (type solid)) (layer "Edge.Cuts"))
 (gr_line (start 36.602629 44.59952) (end 36.6014 44.649107) (stroke (width 0.2) (type solid)) (layer "Edge.Cuts"))
 (gr_line (start 58.272574 43.907806) (end 58.235158 43.875572) (stroke (width 0.2) (type solid)) (layer "Edge.Cuts"))
 (gr_line (start 37.310565 43.692332) (end 37.264226 43.707664) (stroke (width 0.2) (type solid)) (layer "Edge.Cuts"))
 (gr_line (start 36.612359 44.501437) (end 36.606293 44.550269) (stroke (width 0.2) (type solid)) (layer "Edge.Cuts"))
 (gr_line (start 36.631559 67.392859) (end 36.644625 67.439943) (stroke (width 0.2) (type solid)) (layer "Edge.Cuts"))
 (gr_line (start 58.525279 44.266424) (end 58.505518 44.221824) (stroke (width 0.2) (type solid)) (layer "Edge.Cuts"))
 (gr_line (start 58.596506 44.550269) (end 58.59044 44.501437) (stroke (width 0.2) (type solid)) (layer "Edge.Cuts"))
 (gr_line (start 57.700237 68.144214) (end 57.749069 68.138149) (stroke (width 0.2) (type solid)) (layer "Edge.Cuts"))
 (gr_line (start 58.433388 44.094307) (end 58.405176 44.054168) (stroke (width 0.2) (type solid)) (layer "Edge.Cuts"))
 (gr_line (start 37.046599 67.981097) (end 37.087976 68.007247) (stroke (width 0.2) (type solid)) (layer "Edge.Cuts"))
 (gr_line (start 37.310565 68.105883) (end 37.357649 68.118949) (stroke (width 0.2) (type solid)) (layer "Edge.Cuts"))
 (segment (start 39.3572 47.1328) (end 38.5572 47.9328) (width 0.25) (layer "B.Cu") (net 7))
 (segment (start 42.25 48.275) (end 38.8994 48.275) (width 0.25) (layer "B.Cu") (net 7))
 (segment (start 39.3572 45.4308) (end 39.3572 47.1328) (width 0.25) (layer "B.Cu") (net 7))
 (segment (start 38.5572 44.6308) (end 39.3572 45.4308) (width 0.25) (layer "B.Cu") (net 7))
 (segment (start 38.8994 48.275) (end 38.5572 47.9328) (width 0.25) (layer "B.Cu") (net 7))
 (segment (start 48.4982 61.9856) (end 43.784128 61.9856) (width 0.4) (layer "F.Cu") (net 4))
 (segment (start 50.1396 65.3034) (end 50.1396 63.627) (width 0.4) (layer "F.Cu") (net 4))
 (segment (start 47.5964 65.8414) (end 49.6016 65.8414) (width 0.4) (layer "F.Cu") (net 4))
 (segment (start 42.25 60.451472) (end 42.25 57.175) (width 0.4) (layer "F.Cu") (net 4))
 (segment (start 50.1396 63.627) (end 48.4982 61.9856) (width 0.4) (layer "F.Cu") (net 4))
 (segment (start 43.784128 61.9856) (end 42.25 60.451472) (width 0.4) (layer "F.Cu") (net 4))
 (segment (start 46.33 64.575) (end 47.5964 65.8414) (width 0.4) (layer "F.Cu") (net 4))
 (segment (start 49.6016 65.8414) (end 50.1396 65.3034) (width 0.4) (layer "F.Cu") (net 4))
 (segment (start 37.0586 47.8544) (end 37.0586 51.1556) (width 0.4) (layer "B.Cu") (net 4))
 (segment (start 39.4322 55.7898) (end 39.0398 55.3974) (width 0.4) (layer "B.Cu") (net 4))
 (segment (start 37.0586 51.1556) (end 37.2872 50.927) (width 0.4) (layer "B.Cu") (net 4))
 (segment (start 38.4302 59.7408) (end 38.5572 59.6138) (width 0.4) (layer "B.Cu") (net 4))
 (segment (start 38.4302 63.5453) (end 38.4302 59.7408) (width 0.4) (layer "B.Cu") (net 4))
 (segment (start 39.0398 55.3974) (end 38.0238 55.3974) (width 0.4) (layer "B.Cu") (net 4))
 (segment (start 40.9978 62.4332) (end 38.879801 62.4332) (width 0.4) (layer "B.Cu") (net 4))
 (segment (start 38.5572 59.6138) (end 39.4322 58.7388) (width 0.4) (layer "B.Cu") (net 4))
 (segment (start 38.4302 66.4983) (end 38.4059 66.5226) (width 0.4) (layer "B.Cu") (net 4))
 (segment (start 38.0238 55.3974) (end 37.0586 54.4322) (width 0.4) (layer "B.Cu") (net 4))
 (segment (start 38.5572 46.3558) (end 37.0586 47.8544) (width 0.4) (layer "B.Cu") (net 4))
 (segment (start 38.4302 62.882801) (end 38.4302 63.5453) (width 0.4) (layer "B.Cu") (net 4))
 (segment (start 38.5564 49.6578) (end 37.2872 50.927) (width 0.4) (layer "B.Cu") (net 4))
 (segment (start 39.4322 58.7388) (end 39.4322 55.7898) (width 0.4) (layer "B.Cu") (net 4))
 (segment (start 41.8728 63.3082) (end 45.0632 63.3082) (width 0.4) (layer "B.Cu") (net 4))
 (segment (start 38.879801 62.4332) (end 38.4302 62.882801) (width 0.4) (layer "B.Cu") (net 4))
 (segment (start 38.4302 63.5453) (end 38.4302 66.4983) (width 0.4) (layer "B.Cu") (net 4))
 (segment (start 40.9978 62.4332) (end 41.8728 63.3082) (width 0.4) (layer "B.Cu") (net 4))
 (segment (start 37.0586 54.4322) (end 37.0586 51.1556) (width 0.4) (layer "B.Cu") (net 4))
 (segment (start 38.5572 49.6578) (end 38.5564 49.6578) (width 0.4) (layer "B.Cu") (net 4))
 (segment (start 45.0632 63.3082) (end 46.33 64.575) (width 0.4) (layer "B.Cu") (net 4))
 (segment (start 48.87 64.5672) (end 46.8884 62.5856) (width 0.4) (layer "F.Cu") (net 3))
 (segment (start 48.87 64.575) (end 48.87 64.5672) (width 0.4) (layer "F.Cu") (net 3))
 (segment (start 41.2 52.885) (end 42.25 51.835) (width 0.4) (layer "F.Cu") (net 3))
 (segment (start 41.2 60.25) (end 41.2 52.885) (width 0.4) (layer "F.Cu") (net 3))
 (segment (start 46.8884 62.5856) (end 43.5356 62.5856) (width 0.4) (layer "F.Cu") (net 3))
 (segment (start 43.5356 62.5856) (end 41.2 60.25) (width 0.4) (layer "F.Cu") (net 3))
 (segment (start 48.87 64.575) (end 46.9224 66.5226) (width 0.4) (layer "B.Cu") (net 3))
 (segment (start 40.1309 66.5226) (end 39.2559 67.3976) (width 0.4) (layer "B.Cu") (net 3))
 (segment (start 46.9224 66.5226) (end 40.1309 66.5226) (width 0.4) (layer "B.Cu") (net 3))
 (segment (start 37.4684 63.5571) (end 37.4802 63.5453) (width 0.4) (layer "B.Cu") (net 3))
 (segment (start 37.4684 67.0848) (end 37.4684 63.5571) (width 0.4) (layer "B.Cu") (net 3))
 (segment (start 39.3802 63.5453) (end 39.3802 65.7719) (width 0.4) (layer "B.Cu") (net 3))
 (segment (start 37.7812 67.3976) (end 37.4684 67.0848) (width 0.4) (layer "B.Cu") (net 3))
 (segment (start 39.3802 65.7719) (end 40.1309 66.5226) (width 0.4) (layer "B.Cu") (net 3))
 (segment (start 39.2559 67.3976) (end 37.7812 67.3976) (width 0.4) (layer "B.Cu") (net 3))
 (segment (start 37.7572 53.6868) (end 38.5572 54.4868) (width 0.25) (layer "B.Cu") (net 8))
 (segment (start 39.2722 54.4868) (end 40.3098 55.5244) (width 0.25) (layer "B.Cu") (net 8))
 (segment (start 39.3802 61.2703) (end 41.5599 61.2703) (width 0.25) (layer "B.Cu") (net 8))
 (segment (start 40.3098 55.5244) (end 40.3098 60.0202) (width 0.25) (layer "B.Cu") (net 8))
 (segment (start 56.59 59.107) (end 53.2638 62.4332) (width 0.25) (layer "B.Cu") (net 8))
 (segment (start 37.7572 51.9848) (end 37.7572 53.6868) (width 0.25) (layer "B.Cu") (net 8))
 (segment (start 38.5572 54.4868) (end 39.2722 54.4868) (width 0.25) (layer "B.Cu") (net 8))
 (segment (start 38.5572 51.1848) (end 37.7572 51.9848) (width 0.25) (layer "B.Cu") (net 8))
 (segment (start 41.5599 61.2703) (end 42.7228 62.4332) (width 0.25) (layer "B.Cu") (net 8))
 (segment (start 40.3098 60.0202) (end 41.5599 61.2703) (width 0.25) (layer "B.Cu") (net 8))
 (segment (start 42.7228 62.4332) (end 53.2638 62.4332) (width 0.25) (layer "B.Cu") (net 8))
 (segment (start 42.25 50.055) (end 39.687 50.055) (width 0.25) (layer "B.Cu") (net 8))
 (segment (start 56.59 53.9025) (end 56.59 59.107) (width 0.25) (layer "B.Cu") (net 8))
 (segment (start 39.687 50.055) (end 38.5572 51.1848) (width 0.25) (layer "B.Cu") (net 8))
 (segment (start 52.95 56.285) (end 53.95 57.285) (width 0.25) (layer "F.Cu") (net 1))
 (segment (start 53.95 57.285) (end 53.95 64.575) (width 0.25) (layer "F.Cu") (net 1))
 (segment (start 56.7944 54.7894) (end 52.95 50.945) (width 0.25) (layer "F.Cu") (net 2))
 (segment (start 50.5244 66.3664) (end 46.1226 66.3664) (width 0.25) (layer "F.Cu") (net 2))
 (segment (start 56.7944 65.5574) (end 56.7944 54.7894) (width 0.25) (layer "F.Cu") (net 2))
 (segment (start 39.9034 63.9826) (end 39.9034 65.2272) (width 0.25) (layer "F.Cu") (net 2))
 (segment (start 44.5262 63.2714) (end 40.6146 63.2714) (width 0.25) (layer "F.Cu") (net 2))
 (segment (start 51.41 64.575) (end 51.41 65.4808) (width 0.25) (layer "F.Cu") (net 2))
 (segment (start 42.3926 67.7164) (end 54.6354 67.7164) (width 0.25) (layer "F.Cu") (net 2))
 (segment (start 54.6354 67.7164) (end 56.7944 65.5574) (width 0.25) (layer "F.Cu") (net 2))
 (segment (start 40.6146 63.2714) (end 39.9034 63.9826) (width 0.25) (layer "F.Cu") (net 2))
 (segment (start 39.9034 65.2272) (end 42.3926 67.7164) (width 0.25) (layer "F.Cu") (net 2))
 (segment (start 45.0596 65.3034) (end 45.0596 63.8048) (width 0.25) (layer "F.Cu") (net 2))
 (segment (start 45.0596 63.8048) (end 44.5262 63.2714) (width 0.25) (layer "F.Cu") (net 2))
 (segment (start 51.41 65.4808) (end 50.5244 66.3664) (width 0.25) (layer "F.Cu") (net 2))
 (segment (start 46.1226 66.3664) (end 45.0596 65.3034) (width 0.25) (layer "F.Cu") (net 2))
 (segment (start 44.693 66.8164) (end 43.79 65.9134) (width 0.25) (layer "F.Cu") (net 5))
 (segment (start 55.037 56.592) (end 55.037 65.662) (width 0.25) (layer "F.Cu") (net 5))
 (segment (start 55.037 65.662) (end 53.8826 66.8164) (width 0.25) (layer "F.Cu") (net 5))
 (segment (start 52.95 54.505) (end 55.037 56.592) (width 0.25) (layer "F.Cu") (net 5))
 (segment (start 53.8826 66.8164) (end 44.693 66.8164) (width 0.25) (layer "F.Cu") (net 5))
 (segment (start 43.79 65.9134) (end 43.79 64.575) (width 0.25) (layer "F.Cu") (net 5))
 (segment (start 56.1594 55.9344) (end 52.95 52.725) (width 0.25) (layer "F.Cu") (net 6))
 (segment (start 43.9414 67.2664) (end 54.068996 67.2664) (width 0.25) (layer "F.Cu") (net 6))
 (segment (start 41.25 64.575) (end 43.9414 67.2664) (width 0.25) (layer "F.Cu") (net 6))
 (segment (start 56.1594 65.175996) (end 56.1594 55.9344) (width 0.25) (layer "F.Cu") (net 6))
 (segment (start 54.068996 67.2664) (end 56.1594 65.175996) (width 0.25) (layer "F.Cu") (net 6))
 (segment (start 38.5572 53.0098) (end 40.9424 55.395) (width 0.25) (layer "B.Cu") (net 9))
 (segment (start 40.9424 55.395) (end 42.25 55.395) (width 0.25) (layer "B.Cu") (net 9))
 (segment (start 56.59 52.0775) (end 56.59 51.025) (width 0.25) (layer "B.Cu") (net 11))
 (segment (start 52.9621 47.3729) (end 52.95 47.385) (width 0.25) (layer "B.Cu") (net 11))
 (segment (start 56.59 51.025) (end 52.95 47.385) (width 0.25) (layer "B.Cu") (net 11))
 (segment (start 37.4802 61.2703) (end 37.4802 58.8658) (width 0.25) (layer "B.Cu") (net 12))
 (segment (start 38.5572 57.7888) (end 38.5572 56.3118) (width 0.25) (layer "B.Cu") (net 12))
 (segment (start 37.4802 58.8658) (end 38.5572 57.7888) (width 0.25) (layer "B.Cu") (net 12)))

